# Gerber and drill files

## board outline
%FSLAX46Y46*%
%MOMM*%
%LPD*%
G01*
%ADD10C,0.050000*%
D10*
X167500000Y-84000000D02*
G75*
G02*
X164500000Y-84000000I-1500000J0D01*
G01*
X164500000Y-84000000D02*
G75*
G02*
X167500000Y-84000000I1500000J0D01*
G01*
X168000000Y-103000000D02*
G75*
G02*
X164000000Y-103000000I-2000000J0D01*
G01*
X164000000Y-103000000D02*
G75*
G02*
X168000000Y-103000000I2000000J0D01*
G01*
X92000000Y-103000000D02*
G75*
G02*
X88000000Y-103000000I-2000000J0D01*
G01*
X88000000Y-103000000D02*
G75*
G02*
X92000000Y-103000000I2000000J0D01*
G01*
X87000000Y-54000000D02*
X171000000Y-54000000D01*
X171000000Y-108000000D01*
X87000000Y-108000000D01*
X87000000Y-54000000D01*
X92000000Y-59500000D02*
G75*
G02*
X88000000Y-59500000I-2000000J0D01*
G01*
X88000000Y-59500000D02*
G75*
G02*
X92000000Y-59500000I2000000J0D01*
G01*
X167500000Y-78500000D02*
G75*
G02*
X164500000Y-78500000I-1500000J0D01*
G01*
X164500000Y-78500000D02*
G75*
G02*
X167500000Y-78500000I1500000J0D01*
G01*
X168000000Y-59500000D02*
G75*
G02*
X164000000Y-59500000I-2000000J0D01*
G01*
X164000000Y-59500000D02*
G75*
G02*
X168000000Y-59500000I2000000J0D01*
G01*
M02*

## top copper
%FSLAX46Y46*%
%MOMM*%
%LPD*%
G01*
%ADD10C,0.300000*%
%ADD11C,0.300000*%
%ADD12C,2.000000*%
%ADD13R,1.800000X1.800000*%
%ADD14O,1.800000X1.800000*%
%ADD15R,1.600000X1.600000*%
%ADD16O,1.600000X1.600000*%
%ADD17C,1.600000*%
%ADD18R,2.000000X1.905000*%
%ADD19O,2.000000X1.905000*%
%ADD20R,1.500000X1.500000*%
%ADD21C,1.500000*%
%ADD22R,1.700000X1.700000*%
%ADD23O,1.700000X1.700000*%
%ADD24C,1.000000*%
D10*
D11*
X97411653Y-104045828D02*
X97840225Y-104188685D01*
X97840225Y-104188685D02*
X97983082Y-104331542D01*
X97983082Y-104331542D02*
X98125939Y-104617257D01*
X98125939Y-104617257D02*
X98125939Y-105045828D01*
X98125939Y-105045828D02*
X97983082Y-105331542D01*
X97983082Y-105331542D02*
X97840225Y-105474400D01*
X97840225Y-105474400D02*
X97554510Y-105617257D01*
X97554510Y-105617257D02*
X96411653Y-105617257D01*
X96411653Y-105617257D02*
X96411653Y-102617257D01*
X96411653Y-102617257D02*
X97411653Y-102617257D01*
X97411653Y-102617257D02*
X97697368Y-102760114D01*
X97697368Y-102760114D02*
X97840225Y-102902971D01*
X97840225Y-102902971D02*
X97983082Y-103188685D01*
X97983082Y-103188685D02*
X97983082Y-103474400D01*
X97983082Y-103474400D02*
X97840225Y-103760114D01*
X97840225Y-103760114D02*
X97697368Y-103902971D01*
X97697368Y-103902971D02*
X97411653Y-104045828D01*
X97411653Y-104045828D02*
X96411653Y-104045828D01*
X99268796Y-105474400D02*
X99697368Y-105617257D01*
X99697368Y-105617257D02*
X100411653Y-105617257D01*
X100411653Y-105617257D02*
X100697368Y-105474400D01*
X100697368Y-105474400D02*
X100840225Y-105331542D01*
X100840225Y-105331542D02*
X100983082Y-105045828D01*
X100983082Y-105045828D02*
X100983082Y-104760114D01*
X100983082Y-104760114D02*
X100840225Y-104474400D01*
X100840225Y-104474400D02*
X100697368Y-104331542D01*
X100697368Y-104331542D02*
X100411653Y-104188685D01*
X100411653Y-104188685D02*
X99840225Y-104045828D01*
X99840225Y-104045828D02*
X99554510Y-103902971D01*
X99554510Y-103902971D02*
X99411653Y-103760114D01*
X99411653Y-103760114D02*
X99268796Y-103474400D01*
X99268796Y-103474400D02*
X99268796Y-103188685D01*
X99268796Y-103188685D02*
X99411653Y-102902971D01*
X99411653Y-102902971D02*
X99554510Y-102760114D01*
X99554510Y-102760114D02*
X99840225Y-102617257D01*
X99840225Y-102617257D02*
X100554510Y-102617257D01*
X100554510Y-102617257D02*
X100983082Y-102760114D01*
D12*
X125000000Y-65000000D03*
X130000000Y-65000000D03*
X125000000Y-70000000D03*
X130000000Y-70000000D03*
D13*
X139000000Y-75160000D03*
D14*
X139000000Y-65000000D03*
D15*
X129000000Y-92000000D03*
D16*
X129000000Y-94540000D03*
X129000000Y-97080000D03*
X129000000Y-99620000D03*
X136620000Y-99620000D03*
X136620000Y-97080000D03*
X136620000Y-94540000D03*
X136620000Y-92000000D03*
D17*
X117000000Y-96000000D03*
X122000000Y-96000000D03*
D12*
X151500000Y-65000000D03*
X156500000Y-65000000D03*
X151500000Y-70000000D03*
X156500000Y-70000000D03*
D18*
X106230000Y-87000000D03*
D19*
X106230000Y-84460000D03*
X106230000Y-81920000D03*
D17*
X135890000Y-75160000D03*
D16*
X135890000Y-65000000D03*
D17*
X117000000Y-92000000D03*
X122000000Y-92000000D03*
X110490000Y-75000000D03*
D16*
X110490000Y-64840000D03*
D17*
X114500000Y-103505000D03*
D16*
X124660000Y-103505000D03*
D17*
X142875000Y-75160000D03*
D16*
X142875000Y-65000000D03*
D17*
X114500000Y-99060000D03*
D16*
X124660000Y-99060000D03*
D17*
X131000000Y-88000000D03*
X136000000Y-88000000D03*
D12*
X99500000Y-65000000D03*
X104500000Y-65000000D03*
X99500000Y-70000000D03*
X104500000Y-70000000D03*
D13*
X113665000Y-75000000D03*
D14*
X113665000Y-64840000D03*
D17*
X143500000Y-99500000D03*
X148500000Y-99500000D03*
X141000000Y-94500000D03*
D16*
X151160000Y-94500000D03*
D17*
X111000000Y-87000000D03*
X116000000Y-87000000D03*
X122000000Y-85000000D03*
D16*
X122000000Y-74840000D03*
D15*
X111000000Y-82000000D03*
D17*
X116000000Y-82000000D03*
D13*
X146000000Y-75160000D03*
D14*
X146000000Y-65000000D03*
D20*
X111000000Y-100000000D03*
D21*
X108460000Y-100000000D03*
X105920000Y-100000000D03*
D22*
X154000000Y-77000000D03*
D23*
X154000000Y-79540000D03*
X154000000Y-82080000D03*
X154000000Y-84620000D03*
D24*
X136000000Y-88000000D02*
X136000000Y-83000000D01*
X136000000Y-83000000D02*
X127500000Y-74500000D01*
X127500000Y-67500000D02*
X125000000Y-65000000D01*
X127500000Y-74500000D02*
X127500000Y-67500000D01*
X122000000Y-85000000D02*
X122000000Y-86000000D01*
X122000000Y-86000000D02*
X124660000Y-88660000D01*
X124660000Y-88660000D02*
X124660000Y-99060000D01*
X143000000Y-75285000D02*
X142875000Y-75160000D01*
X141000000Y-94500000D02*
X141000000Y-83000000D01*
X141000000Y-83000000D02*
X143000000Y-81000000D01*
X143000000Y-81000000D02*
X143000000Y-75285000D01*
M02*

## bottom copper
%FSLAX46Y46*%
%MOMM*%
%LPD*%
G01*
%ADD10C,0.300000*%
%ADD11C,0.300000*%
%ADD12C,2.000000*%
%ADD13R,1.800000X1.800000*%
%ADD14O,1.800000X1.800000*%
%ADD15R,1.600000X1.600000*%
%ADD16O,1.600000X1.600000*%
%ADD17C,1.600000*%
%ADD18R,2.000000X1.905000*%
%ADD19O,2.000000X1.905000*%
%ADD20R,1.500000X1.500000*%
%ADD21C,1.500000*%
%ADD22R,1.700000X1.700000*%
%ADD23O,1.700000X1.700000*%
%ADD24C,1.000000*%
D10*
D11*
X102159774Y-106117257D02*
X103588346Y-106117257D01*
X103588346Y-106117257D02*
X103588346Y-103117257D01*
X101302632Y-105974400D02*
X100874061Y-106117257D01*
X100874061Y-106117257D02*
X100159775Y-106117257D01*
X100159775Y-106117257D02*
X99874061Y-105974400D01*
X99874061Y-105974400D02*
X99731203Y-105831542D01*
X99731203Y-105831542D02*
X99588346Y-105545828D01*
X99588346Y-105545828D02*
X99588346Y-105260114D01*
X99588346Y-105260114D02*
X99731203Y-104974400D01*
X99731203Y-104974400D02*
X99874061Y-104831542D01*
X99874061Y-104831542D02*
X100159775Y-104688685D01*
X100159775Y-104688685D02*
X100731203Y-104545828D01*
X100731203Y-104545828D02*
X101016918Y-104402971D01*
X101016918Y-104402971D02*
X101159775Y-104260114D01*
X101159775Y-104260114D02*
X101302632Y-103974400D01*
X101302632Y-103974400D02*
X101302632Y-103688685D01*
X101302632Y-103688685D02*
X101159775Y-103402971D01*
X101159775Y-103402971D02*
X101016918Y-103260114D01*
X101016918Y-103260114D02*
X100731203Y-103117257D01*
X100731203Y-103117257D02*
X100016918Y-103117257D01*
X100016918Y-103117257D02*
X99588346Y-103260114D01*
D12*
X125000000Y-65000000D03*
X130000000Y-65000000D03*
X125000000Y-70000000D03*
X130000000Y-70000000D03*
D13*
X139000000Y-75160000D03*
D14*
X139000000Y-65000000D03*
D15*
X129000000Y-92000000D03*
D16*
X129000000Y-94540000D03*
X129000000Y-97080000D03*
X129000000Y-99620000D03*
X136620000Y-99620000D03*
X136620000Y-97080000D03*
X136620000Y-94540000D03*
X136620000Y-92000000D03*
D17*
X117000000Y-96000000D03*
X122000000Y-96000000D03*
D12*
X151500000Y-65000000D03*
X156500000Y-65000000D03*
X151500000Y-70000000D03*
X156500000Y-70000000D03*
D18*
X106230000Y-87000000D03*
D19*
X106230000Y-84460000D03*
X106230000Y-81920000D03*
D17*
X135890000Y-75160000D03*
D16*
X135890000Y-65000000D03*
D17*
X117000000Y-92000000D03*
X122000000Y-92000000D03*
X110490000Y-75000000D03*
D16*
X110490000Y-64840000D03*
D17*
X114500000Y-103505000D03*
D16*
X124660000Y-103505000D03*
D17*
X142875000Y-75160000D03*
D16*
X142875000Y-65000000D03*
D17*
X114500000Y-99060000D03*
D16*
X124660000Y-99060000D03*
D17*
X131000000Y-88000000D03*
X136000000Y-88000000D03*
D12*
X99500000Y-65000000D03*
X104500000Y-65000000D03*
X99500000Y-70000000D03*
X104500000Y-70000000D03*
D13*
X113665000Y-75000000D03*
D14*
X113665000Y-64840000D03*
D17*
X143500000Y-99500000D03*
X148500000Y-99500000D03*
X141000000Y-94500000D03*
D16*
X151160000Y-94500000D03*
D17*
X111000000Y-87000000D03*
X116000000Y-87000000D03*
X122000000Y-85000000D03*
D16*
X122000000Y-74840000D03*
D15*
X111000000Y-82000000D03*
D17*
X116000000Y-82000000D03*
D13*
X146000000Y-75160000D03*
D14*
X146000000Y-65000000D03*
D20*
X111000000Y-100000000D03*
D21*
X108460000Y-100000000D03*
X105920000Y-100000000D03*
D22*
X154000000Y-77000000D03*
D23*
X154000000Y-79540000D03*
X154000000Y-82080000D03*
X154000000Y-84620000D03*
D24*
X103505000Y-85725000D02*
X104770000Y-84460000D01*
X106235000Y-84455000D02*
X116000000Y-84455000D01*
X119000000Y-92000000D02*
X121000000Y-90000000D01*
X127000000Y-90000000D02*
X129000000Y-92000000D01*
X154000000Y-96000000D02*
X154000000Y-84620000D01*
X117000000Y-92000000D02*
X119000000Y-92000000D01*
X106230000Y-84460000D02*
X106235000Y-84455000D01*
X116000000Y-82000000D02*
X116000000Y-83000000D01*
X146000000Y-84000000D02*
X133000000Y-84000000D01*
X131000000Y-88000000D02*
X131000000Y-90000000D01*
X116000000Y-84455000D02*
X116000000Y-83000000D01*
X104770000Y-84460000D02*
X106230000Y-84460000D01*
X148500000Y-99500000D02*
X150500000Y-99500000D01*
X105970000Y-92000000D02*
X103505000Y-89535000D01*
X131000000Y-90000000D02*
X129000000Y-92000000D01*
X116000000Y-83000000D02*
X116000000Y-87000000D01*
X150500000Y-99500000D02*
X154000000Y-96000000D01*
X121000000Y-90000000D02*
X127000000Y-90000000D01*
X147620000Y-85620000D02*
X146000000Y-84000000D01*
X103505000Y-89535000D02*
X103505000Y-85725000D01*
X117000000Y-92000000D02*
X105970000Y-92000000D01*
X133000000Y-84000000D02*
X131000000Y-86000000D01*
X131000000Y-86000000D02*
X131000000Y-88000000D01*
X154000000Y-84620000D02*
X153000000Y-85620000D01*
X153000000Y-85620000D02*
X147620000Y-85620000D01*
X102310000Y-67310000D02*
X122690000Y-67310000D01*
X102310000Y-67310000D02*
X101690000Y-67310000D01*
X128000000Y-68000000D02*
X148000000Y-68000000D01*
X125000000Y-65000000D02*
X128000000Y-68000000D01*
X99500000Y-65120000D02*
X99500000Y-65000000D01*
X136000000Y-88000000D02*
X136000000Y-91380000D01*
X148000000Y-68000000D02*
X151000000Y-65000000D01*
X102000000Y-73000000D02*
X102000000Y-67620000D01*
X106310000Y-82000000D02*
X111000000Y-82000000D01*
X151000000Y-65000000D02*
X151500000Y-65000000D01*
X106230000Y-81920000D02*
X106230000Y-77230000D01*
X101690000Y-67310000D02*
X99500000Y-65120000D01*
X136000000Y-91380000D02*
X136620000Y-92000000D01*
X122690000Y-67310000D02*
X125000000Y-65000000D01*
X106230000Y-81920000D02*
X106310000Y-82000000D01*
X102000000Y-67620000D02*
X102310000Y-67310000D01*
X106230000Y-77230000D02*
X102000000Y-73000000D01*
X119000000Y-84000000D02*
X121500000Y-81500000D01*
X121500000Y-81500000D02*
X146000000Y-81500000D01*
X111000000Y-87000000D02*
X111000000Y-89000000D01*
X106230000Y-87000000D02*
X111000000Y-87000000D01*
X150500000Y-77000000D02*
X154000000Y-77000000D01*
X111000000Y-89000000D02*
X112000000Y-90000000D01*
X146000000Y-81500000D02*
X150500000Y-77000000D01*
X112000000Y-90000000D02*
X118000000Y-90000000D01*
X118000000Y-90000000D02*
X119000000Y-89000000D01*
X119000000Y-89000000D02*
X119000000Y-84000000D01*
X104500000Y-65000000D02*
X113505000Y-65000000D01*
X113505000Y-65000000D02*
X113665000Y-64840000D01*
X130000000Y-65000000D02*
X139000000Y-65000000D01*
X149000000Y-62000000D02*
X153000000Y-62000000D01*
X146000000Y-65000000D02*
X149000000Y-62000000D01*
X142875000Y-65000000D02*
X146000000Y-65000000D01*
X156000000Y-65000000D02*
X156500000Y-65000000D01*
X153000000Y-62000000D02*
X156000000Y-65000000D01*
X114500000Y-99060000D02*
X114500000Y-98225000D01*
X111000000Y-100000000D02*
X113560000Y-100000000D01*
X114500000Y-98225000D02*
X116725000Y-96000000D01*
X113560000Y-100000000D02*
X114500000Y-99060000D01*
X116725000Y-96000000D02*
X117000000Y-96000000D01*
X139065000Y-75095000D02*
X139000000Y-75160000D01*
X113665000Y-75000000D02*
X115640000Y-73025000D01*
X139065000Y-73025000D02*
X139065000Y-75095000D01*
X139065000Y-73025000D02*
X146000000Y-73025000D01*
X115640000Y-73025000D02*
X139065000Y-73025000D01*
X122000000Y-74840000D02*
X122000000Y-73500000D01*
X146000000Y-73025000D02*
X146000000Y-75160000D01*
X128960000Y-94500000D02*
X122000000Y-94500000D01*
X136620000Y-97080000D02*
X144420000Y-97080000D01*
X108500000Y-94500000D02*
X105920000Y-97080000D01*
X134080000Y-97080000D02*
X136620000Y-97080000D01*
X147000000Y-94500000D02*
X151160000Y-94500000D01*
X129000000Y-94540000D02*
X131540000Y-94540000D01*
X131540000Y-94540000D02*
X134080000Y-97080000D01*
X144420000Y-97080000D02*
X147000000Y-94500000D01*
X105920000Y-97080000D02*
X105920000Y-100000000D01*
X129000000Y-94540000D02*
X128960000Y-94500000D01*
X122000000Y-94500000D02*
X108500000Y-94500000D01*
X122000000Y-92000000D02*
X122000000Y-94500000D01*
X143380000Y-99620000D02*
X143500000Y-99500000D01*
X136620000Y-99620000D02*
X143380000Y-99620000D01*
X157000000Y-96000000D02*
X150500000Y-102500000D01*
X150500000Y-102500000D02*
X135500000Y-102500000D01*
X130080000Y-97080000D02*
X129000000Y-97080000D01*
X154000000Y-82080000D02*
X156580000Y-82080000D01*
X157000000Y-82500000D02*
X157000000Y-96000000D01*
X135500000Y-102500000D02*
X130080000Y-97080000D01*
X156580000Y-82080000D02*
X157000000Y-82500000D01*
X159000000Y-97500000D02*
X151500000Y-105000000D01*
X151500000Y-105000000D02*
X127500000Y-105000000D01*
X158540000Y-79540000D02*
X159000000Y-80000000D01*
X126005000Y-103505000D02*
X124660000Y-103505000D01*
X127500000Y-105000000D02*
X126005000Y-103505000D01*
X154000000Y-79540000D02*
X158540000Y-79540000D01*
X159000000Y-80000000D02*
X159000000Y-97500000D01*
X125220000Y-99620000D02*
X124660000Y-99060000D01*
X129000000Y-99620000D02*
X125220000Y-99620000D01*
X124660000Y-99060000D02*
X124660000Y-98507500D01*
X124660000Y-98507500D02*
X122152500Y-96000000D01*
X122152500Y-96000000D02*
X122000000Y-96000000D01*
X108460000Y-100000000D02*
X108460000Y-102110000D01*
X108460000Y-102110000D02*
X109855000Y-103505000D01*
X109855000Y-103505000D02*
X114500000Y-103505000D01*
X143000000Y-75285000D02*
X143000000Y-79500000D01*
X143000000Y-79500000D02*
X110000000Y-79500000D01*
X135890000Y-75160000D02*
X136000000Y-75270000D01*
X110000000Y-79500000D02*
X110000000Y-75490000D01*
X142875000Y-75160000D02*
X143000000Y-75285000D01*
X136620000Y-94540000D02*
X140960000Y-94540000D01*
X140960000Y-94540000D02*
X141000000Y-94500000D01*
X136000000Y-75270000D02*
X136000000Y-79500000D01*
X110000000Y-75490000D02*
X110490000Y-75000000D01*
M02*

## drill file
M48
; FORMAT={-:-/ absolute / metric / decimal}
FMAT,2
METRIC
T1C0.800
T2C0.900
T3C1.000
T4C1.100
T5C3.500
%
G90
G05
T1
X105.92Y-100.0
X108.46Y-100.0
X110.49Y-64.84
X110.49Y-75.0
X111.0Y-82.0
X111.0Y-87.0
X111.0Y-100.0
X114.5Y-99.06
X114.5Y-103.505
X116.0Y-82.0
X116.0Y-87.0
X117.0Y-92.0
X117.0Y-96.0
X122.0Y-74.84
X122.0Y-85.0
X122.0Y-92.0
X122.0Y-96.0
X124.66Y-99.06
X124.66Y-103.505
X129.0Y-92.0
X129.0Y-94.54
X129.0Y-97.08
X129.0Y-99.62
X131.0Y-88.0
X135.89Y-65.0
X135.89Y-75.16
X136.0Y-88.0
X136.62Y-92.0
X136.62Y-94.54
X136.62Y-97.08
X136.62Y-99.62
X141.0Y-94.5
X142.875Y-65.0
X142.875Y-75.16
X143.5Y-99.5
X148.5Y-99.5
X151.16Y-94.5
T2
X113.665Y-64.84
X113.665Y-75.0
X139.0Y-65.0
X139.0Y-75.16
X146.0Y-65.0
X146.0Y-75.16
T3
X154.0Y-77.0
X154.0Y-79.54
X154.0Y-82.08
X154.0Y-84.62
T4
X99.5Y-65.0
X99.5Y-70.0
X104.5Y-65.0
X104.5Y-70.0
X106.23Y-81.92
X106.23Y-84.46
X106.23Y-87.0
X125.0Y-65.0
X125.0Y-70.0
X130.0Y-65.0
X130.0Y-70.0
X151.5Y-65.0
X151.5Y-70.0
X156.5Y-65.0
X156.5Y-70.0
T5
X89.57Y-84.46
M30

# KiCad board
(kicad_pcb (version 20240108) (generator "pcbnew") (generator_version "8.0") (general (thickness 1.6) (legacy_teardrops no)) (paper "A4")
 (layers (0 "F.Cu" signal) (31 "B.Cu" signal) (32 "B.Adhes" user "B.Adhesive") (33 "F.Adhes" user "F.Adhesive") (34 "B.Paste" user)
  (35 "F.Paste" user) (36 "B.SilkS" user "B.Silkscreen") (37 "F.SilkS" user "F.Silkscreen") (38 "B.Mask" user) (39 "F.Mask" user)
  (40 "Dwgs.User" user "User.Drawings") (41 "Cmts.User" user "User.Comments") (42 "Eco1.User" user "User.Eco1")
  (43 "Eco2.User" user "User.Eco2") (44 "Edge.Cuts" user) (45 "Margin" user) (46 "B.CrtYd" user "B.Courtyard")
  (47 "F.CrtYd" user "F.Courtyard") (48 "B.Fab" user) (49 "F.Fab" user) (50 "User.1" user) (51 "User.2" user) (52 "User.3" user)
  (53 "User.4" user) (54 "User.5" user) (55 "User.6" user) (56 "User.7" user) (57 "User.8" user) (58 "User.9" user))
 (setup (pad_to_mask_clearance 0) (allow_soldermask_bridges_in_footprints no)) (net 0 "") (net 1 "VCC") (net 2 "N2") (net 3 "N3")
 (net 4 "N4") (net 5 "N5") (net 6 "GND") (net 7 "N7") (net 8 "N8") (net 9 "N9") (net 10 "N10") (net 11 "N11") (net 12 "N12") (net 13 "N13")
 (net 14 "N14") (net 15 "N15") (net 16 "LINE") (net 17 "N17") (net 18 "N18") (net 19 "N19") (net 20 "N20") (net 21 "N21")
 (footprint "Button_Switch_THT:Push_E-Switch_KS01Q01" (layer "F.Cu") (at 125 65)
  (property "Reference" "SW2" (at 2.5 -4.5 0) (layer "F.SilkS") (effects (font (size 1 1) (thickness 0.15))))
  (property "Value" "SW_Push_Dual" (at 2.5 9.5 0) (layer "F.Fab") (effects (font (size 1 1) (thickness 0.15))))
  (pad "1" thru_hole circle (at 0 0) (size 2 2) (drill 1.1) (layers "*.Cu" "*.Mask") (remove_unused_layers no) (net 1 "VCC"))
  (pad "2" thru_hole circle (at 5 0) (size 2 2) (drill 1.1) (layers "*.Cu" "*.Mask") (remove_unused_layers no) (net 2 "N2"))
  (pad "3" thru_hole circle (at 0 5) (size 2 2) (drill 1.1) (layers "*.Cu" "*.Mask") (remove_unused_layers no) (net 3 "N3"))
  (pad "4" thru_hole circle (at 5 5) (size 2 2) (drill 1.1) (layers "*.Cu" "*.Mask") (remove_unused_layers no) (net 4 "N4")))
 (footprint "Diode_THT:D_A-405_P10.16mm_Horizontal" (layer "F.Cu") (at 139 75.16 90)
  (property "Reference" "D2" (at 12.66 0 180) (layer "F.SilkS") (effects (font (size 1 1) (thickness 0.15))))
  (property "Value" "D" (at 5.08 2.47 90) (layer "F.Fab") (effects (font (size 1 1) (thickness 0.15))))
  (pad "1" thru_hole rect (at 0 0 90) (size 1.8 1.8) (drill 0.9) (layers "*.Cu" "*.Mask") (remove_unused_layers no) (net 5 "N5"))
  (pad "2" thru_hole oval (at 10.16 0 90) (size 1.8 1.8) (drill 0.9) (layers "*.Cu" "*.Mask") (remove_unused_layers no) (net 2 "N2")))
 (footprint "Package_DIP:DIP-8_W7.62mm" (layer "F.Cu") (at 129 92)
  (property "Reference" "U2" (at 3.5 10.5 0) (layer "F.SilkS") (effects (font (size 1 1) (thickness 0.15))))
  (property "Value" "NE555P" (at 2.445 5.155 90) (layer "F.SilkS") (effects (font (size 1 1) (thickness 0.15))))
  (pad "1" thru_hole rect (at 0 0) (size 1.6 1.6) (drill 0.8) (layers "*.Cu" "*.Mask") (remove_unused_layers no) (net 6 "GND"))
  (pad "2" thru_hole oval (at 0 2.54) (size 1.6 1.6) (drill 0.8) (layers "*.Cu" "*.Mask") (remove_unused_layers no) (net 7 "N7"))
  (pad "3" thru_hole oval (at 0 5.08) (size 1.6 1.6) (drill 0.8) (layers "*.Cu" "*.Mask") (remove_unused_layers no) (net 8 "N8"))
  (pad "4" thru_hole oval (at 0 7.62) (size 1.6 1.6) (drill 0.8) (layers "*.Cu" "*.Mask") (remove_unused_layers no) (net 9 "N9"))
  (pad "5" thru_hole oval (at 7.62 7.62) (size 1.6 1.6) (drill 0.8) (layers "*.Cu" "*.Mask") (remove_unused_layers no) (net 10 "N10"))
  (pad "6" thru_hole oval (at 7.62 5.08) (size 1.6 1.6) (drill 0.8) (layers "*.Cu" "*.Mask") (remove_unused_layers no) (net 7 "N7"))
  (pad "7" thru_hole oval (at 7.62 2.54) (size 1.6 1.6) (drill 0.8) (layers "*.Cu" "*.Mask") (remove_unused_layers no) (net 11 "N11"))
  (pad "8" thru_hole oval (at 7.62 0) (size 1.6 1.6) (drill 0.8) (layers "*.Cu" "*.Mask") (remove_unused_layers no) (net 1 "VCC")))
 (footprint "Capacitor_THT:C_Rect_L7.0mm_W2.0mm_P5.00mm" (layer "F.Cu") (at 117 96)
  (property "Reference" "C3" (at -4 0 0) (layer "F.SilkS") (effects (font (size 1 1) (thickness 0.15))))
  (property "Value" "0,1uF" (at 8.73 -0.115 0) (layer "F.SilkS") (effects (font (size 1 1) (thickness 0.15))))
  (pad "1" thru_hole circle (at 0 0) (size 1.6 1.6) (drill 0.8) (layers "*.Cu" "*.Mask") (remove_unused_layers no) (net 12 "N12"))
  (pad "2" thru_hole circle (at 5 0) (size 1.6 1.6) (drill 0.8) (layers "*.Cu" "*.Mask") (remove_unused_layers no) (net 9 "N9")))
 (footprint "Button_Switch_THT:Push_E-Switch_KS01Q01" (layer "F.Cu") (at 151.5 65)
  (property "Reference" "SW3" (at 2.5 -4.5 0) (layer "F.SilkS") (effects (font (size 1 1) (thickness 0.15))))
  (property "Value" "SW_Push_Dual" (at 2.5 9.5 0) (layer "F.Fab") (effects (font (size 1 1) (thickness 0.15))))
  (pad "1" thru_hole circle (at 0 0) (size 2 2) (drill 1.1) (layers "*.Cu" "*.Mask") (remove_unused_layers no) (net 1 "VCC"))
  (pad "2" thru_hole circle (at 5 0) (size 2 2) (drill 1.1) (layers "*.Cu" "*.Mask") (remove_unused_layers no) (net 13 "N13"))
  (pad "3" thru_hole circle (at 0 5) (size 2 2) (drill 1.1) (layers "*.Cu" "*.Mask") (remove_unused_layers no) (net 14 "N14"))
  (pad "4" thru_hole circle (at 5 5) (size 2 2) (drill 1.1) (layers "*.Cu" "*.Mask") (remove_unused_layers no) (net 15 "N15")))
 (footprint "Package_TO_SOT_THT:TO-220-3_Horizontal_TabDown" (layer "F.Cu") (at 106.23 87 90)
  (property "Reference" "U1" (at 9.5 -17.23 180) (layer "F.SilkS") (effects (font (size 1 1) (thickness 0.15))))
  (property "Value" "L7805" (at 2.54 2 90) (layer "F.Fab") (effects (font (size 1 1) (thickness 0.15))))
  (pad "" np_thru_hole circle (at 2.54 -16.66 90) (size 3.5 3.5) (drill 3.5) (layers "*.Cu" "*.Mask"))
  (pad "1" thru_hole rect (at 0 0 90) (size 1.905 2) (drill 1.1) (layers "*.Cu" "*.Mask") (remove_unused_layers no) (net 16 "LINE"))
  (pad "2" thru_hole oval (at 2.54 0 90) (size 1.905 2) (drill 1.1) (layers "*.Cu" "*.Mask") (remove_unused_layers no) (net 6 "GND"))
  (pad "3" thru_hole oval (at 5.08 0 90) (size 1.905 2) (drill 1.1) (layers "*.Cu" "*.Mask") (remove_unused_layers no) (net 1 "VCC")))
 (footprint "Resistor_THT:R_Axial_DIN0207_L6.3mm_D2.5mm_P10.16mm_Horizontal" (layer "F.Cu") (at 135.89 75.16 90)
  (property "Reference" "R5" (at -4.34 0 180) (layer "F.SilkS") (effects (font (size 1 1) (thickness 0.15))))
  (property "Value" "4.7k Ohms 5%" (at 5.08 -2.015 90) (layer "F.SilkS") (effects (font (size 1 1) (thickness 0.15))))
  (pad "1" thru_hole circle (at 0 0 90) (size 1.6 1.6) (drill 0.8) (layers "*.Cu" "*.Mask") (remove_unused_layers no) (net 11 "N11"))
  (pad "2" thru_hole oval (at 10.16 0 90) (size 1.6 1.6) (drill 0.8) (layers "*.Cu" "*.Mask") (remove_unused_layers no) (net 2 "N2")))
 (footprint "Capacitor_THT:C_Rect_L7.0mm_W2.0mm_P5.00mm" (layer "F.Cu") (at 117 92)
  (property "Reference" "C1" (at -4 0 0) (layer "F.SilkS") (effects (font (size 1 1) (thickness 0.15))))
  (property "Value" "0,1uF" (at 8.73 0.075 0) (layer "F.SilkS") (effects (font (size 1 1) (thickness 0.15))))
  (pad "1" thru_hole circle (at 0 0) (size 1.6 1.6) (drill 0.8) (layers "*.Cu" "*.Mask") (remove_unused_layers no) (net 6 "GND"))
  (pad "2" thru_hole circle (at 5 0) (size 1.6 1.6) (drill 0.8) (layers "*.Cu" "*.Mask") (remove_unused_layers no) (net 7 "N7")))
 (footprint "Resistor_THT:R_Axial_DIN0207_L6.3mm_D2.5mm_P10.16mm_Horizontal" (layer "F.Cu") (at 110.49 75 90)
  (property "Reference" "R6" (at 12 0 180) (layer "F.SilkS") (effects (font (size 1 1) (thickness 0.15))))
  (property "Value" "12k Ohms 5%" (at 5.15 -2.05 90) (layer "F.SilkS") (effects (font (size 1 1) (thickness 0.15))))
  (pad "1" thru_hole circle (at 0 0 90) (size 1.6 1.6) (drill 0.8) (layers "*.Cu" "*.Mask") (remove_unused_layers no) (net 11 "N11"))
  (pad "2" thru_hole oval (at 10.16 0 90) (size 1.6 1.6) (drill 0.8) (layers "*.Cu" "*.Mask") (remove_unused_layers no) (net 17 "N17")))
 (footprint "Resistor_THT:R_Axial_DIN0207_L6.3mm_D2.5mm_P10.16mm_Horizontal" (layer "F.Cu") (at 114.5 103.505)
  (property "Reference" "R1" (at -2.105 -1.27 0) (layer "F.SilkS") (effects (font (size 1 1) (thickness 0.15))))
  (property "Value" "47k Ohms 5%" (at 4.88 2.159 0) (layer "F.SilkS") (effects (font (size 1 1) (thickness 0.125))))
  (pad "1" thru_hole circle (at 0 0) (size 1.6 1.6) (drill 0.8) (layers "*.Cu" "*.Mask") (remove_unused_layers no) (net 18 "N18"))
  (pad "2" thru_hole oval (at 10.16 0) (size 1.6 1.6) (drill 0.8) (layers "*.Cu" "*.Mask") (remove_unused_layers no) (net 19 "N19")))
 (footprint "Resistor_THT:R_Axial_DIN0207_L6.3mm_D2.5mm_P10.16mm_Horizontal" (layer "F.Cu") (at 142.875 75.16 90)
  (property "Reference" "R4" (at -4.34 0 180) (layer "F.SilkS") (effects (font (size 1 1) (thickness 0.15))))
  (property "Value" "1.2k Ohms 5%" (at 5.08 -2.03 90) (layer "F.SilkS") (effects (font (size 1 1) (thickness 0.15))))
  (pad "1" thru_hole circle (at 0 0 90) (size 1.6 1.6) (drill 0.8) (layers "*.Cu" "*.Mask") (remove_unused_layers no) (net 11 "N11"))
  (pad "2" thru_hole oval (at 10.16 0 90) (size 1.6 1.6) (drill 0.8) (layers "*.Cu" "*.Mask") (remove_unused_layers no) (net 13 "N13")))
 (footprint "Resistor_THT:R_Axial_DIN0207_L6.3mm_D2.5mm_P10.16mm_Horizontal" (layer "F.Cu") (at 114.5 99.06)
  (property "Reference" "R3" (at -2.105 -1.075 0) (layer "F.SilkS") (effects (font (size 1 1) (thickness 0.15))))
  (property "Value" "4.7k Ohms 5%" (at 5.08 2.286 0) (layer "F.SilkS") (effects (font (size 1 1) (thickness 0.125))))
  (pad "1" thru_hole circle (at 0 0) (size 1.6 1.6) (drill 0.8) (layers "*.Cu" "*.Mask") (remove_unused_layers no) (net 12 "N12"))
  (pad "2" thru_hole oval (at 10.16 0) (size 1.6 1.6) (drill 0.8) (layers "*.Cu" "*.Mask") (remove_unused_layers no) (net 9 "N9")))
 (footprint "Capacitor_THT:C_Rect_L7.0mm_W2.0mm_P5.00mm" (layer "F.Cu") (at 131 88)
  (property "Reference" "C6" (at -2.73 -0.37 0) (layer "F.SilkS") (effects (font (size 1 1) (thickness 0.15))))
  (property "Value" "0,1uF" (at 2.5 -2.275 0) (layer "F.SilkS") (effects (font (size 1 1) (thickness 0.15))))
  (pad "1" thru_hole circle (at 0 0) (size 1.6 1.6) (drill 0.8) (layers "*.Cu" "*.Mask") (remove_unused_layers no) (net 6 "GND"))
  (pad "2" thru_hole circle (at 5 0) (size 1.6 1.6) (drill 0.8) (layers "*.Cu" "*.Mask") (remove_unused_layers no) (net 1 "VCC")))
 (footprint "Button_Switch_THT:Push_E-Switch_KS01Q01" (layer "F.Cu") (at 99.5 65)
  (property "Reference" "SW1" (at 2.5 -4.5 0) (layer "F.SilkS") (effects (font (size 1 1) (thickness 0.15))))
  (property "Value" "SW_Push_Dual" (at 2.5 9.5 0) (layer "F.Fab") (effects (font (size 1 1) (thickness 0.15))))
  (pad "1" thru_hole circle (at 0 0) (size 2 2) (drill 1.1) (layers "*.Cu" "*.Mask") (remove_unused_layers no) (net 1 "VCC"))
  (pad "2" thru_hole circle (at 5 0) (size 2 2) (drill 1.1) (layers "*.Cu" "*.Mask") (remove_unused_layers no) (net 17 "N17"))
  (pad "3" thru_hole circle (at 0 5) (size 2 2) (drill 1.1) (layers "*.Cu" "*.Mask") (remove_unused_layers no) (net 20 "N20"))
  (pad "4" thru_hole circle (at 5 5) (size 2 2) (drill 1.1) (layers "*.Cu" "*.Mask") (remove_unused_layers no) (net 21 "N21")))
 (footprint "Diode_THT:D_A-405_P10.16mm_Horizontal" (layer "F.Cu") (at 113.665 75 90)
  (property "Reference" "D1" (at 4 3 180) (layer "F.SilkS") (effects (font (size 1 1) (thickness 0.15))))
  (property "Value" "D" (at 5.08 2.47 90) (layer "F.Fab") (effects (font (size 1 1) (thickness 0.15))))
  (pad "1" thru_hole rect (at 0 0 90) (size 1.8 1.8) (drill 0.9) (layers "*.Cu" "*.Mask") (remove_unused_layers no) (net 5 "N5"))
  (pad "2" thru_hole oval (at 10.16 0 90) (size 1.8 1.8) (drill 0.9) (layers "*.Cu" "*.Mask") (remove_unused_layers no) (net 17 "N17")))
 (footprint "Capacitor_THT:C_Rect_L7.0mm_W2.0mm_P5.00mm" (layer "F.Cu") (at 143.5 99.5)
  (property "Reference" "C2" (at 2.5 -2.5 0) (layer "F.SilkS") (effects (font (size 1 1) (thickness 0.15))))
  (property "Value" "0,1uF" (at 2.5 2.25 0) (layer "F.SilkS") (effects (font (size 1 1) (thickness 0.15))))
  (pad "1" thru_hole circle (at 0 0) (size 1.6 1.6) (drill 0.8) (layers "*.Cu" "*.Mask") (remove_unused_layers no) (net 10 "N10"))
  (pad "2" thru_hole circle (at 5 0) (size 1.6 1.6) (drill 0.8) (layers "*.Cu" "*.Mask") (remove_unused_layers no) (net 6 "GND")))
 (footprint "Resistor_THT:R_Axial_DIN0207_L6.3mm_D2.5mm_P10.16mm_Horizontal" (layer "F.Cu") (at 141 94.5)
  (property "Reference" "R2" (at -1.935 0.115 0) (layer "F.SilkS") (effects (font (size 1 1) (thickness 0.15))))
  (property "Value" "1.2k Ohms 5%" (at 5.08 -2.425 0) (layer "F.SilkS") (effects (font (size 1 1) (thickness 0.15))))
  (pad "1" thru_hole circle (at 0 0) (size 1.6 1.6) (drill 0.8) (layers "*.Cu" "*.Mask") (remove_unused_layers no) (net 11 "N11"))
  (pad "2" thru_hole oval (at 10.16 0) (size 1.6 1.6) (drill 0.8) (layers "*.Cu" "*.Mask") (remove_unused_layers no) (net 7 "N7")))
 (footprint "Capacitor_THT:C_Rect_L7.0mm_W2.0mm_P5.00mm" (layer "F.Cu") (at 111 87)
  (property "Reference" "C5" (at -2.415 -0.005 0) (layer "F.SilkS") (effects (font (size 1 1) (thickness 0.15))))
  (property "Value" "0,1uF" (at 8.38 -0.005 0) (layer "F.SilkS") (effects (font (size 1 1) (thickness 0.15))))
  (pad "1" thru_hole circle (at 0 0) (size 1.6 1.6) (drill 0.8) (layers "*.Cu" "*.Mask") (remove_unused_layers no) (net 16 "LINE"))
  (pad "2" thru_hole circle (at 5 0) (size 1.6 1.6) (drill 0.8) (layers "*.Cu" "*.Mask") (remove_unused_layers no) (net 6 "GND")))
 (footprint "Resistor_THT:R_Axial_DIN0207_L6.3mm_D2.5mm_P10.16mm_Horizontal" (layer "F.Cu") (at 122 85 90)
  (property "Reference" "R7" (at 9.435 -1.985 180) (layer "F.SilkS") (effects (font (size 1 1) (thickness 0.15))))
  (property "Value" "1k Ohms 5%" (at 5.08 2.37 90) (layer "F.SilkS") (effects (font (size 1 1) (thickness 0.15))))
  (pad "1" thru_hole circle (at 0 0 90) (size 1.6 1.6) (drill 0.8) (layers "*.Cu" "*.Mask") (remove_unused_layers no) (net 9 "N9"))
  (pad "2" thru_hole oval (at 10.16 0 90) (size 1.6 1.6) (drill 0.8) (layers "*.Cu" "*.Mask") (remove_unused_layers no) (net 5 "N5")))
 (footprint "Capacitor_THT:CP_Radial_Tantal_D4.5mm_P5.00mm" (layer "F.Cu") (at 111 82)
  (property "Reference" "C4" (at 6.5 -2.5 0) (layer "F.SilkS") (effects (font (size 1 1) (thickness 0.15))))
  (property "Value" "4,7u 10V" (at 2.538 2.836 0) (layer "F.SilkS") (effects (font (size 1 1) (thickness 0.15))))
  (pad "1" thru_hole rect (at 0 0) (size 1.6 1.6) (drill 0.8) (layers "*.Cu" "*.Mask") (remove_unused_layers no) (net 1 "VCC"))
  (pad "2" thru_hole circle (at 5 0) (size 1.6 1.6) (drill 0.8) (layers "*.Cu" "*.Mask") (remove_unused_layers no) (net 6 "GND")))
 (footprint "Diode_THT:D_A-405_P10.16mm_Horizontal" (layer "F.Cu") (at 146 75.16 90)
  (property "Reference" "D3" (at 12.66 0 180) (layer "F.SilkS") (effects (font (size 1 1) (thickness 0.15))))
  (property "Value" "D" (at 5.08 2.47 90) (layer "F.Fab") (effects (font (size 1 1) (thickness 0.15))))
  (pad "1" thru_hole rect (at 0 0 90) (size 1.8 1.8) (drill 0.9) (layers "*.Cu" "*.Mask") (remove_unused_layers no) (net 5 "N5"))
  (pad "2" thru_hole oval (at 10.16 0 90) (size 1.8 1.8) (drill 0.9) (layers "*.Cu" "*.Mask") (remove_unused_layers no) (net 13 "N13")))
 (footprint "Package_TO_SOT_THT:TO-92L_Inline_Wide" (layer "F.Cu") (at 111 100 180)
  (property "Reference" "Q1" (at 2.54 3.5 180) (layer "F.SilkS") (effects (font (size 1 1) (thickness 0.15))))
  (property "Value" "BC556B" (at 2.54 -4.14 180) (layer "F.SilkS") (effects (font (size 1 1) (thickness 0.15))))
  (pad "1" thru_hole rect (at 0 0 180) (size 1.5 1.5) (drill 0.8) (layers "*.Cu" "*.Mask") (remove_unused_layers no) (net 12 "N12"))
  (pad "2" thru_hole circle (at 2.54 0 180) (size 1.5 1.5) (drill 0.8) (layers "*.Cu" "*.Mask") (remove_unused_layers no) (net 18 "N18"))
  (pad "3" thru_hole circle (at 5.08 0 180) (size 1.5 1.5) (drill 0.8) (layers "*.Cu" "*.Mask") (remove_unused_layers no) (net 7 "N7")))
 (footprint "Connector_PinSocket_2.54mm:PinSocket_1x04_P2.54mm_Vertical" (layer "F.Cu") (at 154 77)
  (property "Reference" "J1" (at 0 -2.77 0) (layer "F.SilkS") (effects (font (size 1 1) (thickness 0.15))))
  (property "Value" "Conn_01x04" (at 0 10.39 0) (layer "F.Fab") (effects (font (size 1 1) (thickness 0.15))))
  (pad "1" thru_hole rect (at 0 0) (size 1.7 1.7) (drill 1) (layers "*.Cu" "*.Mask") (remove_unused_layers no) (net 16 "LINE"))
  (pad "2" thru_hole oval (at 0 2.54) (size 1.7 1.7) (drill 1) (layers "*.Cu" "*.Mask") (remove_unused_layers no) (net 19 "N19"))
  (pad "3" thru_hole oval (at 0 5.08) (size 1.7 1.7) (drill 1) (layers "*.Cu" "*.Mask") (remove_unused_layers no) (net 8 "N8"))
  (pad "4" thru_hole oval (at 0 7.62) (size 1.7 1.7) (drill 1) (layers "*.Cu" "*.Mask") (remove_unused_layers no) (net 6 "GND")))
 (gr_circle (center 166 84) (end 167.5 84) (stroke (width 0.05) (type default)) (fill none) (layer "Edge.Cuts"))
 (gr_circle (center 166 103) (end 166 101) (stroke (width 0.05) (type default)) (fill none) (layer "Edge.Cuts"))
 (gr_circle (center 90 103) (end 90 101) (stroke (width 0.05) (type default)) (fill none) (layer "Edge.Cuts"))
 (gr_rect (start 87 54) (end 171 108) (stroke (width 0.05) (type default)) (fill none) (layer "Edge.Cuts"))
 (gr_circle (center 90 59.5) (end 90 57.5) (stroke (width 0.05) (type default)) (fill none) (layer "Edge.Cuts"))
 (gr_circle (center 166 78.5) (end 167.5 78.5) (stroke (width 0.05) (type default)) (fill none) (layer "Edge.Cuts"))
 (gr_circle (center 166 59.5) (end 166 57.5) (stroke (width 0.05) (type default)) (fill none) (layer "Edge.Cuts"))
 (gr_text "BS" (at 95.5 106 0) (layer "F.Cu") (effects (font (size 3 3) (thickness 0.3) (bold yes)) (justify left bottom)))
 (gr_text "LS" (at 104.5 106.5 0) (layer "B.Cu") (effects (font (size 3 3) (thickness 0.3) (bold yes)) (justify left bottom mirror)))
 (segment (start 103.505 85.725) (end 104.77 84.46) (width 1) (layer "B.Cu") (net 6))
 (segment (start 106.235 84.455) (end 116 84.455) (width 1) (layer "B.Cu") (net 6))
 (segment (start 119 92) (end 121 90) (width 1) (layer "B.Cu") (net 6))
 (segment (start 127 90) (end 129 92) (width 1) (layer "B.Cu") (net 6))
 (segment (start 154 96) (end 154 84.62) (width 1) (layer "B.Cu") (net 6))
 (segment (start 117 92) (end 119 92) (width 1) (layer "B.Cu") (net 6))
 (segment (start 106.23 84.46) (end 106.235 84.455) (width 1) (layer "B.Cu") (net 6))
 (segment (start 116 82) (end 116 83) (width 1) (layer "B.Cu") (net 6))
 (segment (start 146 84) (end 133 84) (width 1) (layer "B.Cu") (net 6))
 (segment (start 131 88) (end 131 90) (width 1) (layer "B.Cu") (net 6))
 (segment (start 116 84.455) (end 116 83) (width 1) (layer "B.Cu") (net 6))
 (segment (start 104.77 84.46) (end 106.23 84.46) (width 1) (layer "B.Cu") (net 6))
 (segment (start 148.5 99.5) (end 150.5 99.5) (width 1) (layer "B.Cu") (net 6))
 (segment (start 105.97 92) (end 103.505 89.535) (width 1) (layer "B.Cu") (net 6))
 (segment (start 131 90) (end 129 92) (width 1) (layer "B.Cu") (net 6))
 (segment (start 116 83) (end 116 87) (width 1) (layer "B.Cu") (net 6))
 (segment (start 150.5 99.5) (end 154 96) (width 1) (layer "B.Cu") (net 6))
 (segment (start 121 90) (end 127 90) (width 1) (layer "B.Cu") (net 6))
 (segment (start 147.62 85.62) (end 146 84) (width 1) (layer "B.Cu") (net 6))
 (segment (start 103.505 89.535) (end 103.505 85.725) (width 1) (layer "B.Cu") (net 6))
 (segment (start 117 92) (end 105.97 92) (width 1) (layer "B.Cu") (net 6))
 (segment (start 133 84) (end 131 86) (width 1) (layer "B.Cu") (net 6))
 (segment (start 131 86) (end 131 88) (width 1) (layer "B.Cu") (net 6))
 (segment (start 154 84.62) (end 153 85.62) (width 1) (layer "B.Cu") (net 6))
 (segment (start 153 85.62) (end 147.62 85.62) (width 1) (layer "B.Cu") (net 6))
 (segment (start 136 88) (end 136 83) (width 1) (layer "F.Cu") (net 1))
 (segment (start 136 83) (end 127.5 74.5) (width 1) (layer "F.Cu") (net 1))
 (segment (start 127.5 67.5) (end 125 65) (width 1) (layer "F.Cu") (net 1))
 (segment (start 127.5 74.5) (end 127.5 67.5) (width 1) (layer "F.Cu") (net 1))
 (segment (start 102.31 67.31) (end 122.69 67.31) (width 1) (layer "B.Cu") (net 1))
 (segment (start 102.31 67.31) (end 101.69 67.31) (width 1) (layer "B.Cu") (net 1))
 (segment (start 128 68) (end 148 68) (width 1) (layer "B.Cu") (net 1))
 (segment (start 125 65) (end 128 68) (width 1) (layer "B.Cu") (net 1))
 (segment (start 99.5 65.12) (end 99.5 65) (width 1) (layer "B.Cu") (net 1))
 (segment (start 136 88) (end 136 91.38) (width 1) (layer "B.Cu") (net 1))
 (segment (start 148 68) (end 151 65) (width 1) (layer "B.Cu") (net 1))
 (segment (start 102 73) (end 102 67.62) (width 1) (layer "B.Cu") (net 1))
 (segment (start 106.31 82) (end 111 82) (width 1) (layer "B.Cu") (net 1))
 (segment (start 151 65) (end 151.5 65) (width 1) (layer "B.Cu") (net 1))
 (segment (start 106.23 81.92) (end 106.23 77.23) (width 1) (layer "B.Cu") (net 1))
 (segment (start 101.69 67.31) (end 99.5 65.12) (width 1) (layer "B.Cu") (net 1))
 (segment (start 136 91.38) (end 136.62 92) (width 1) (layer "B.Cu") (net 1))
 (segment (start 122.69 67.31) (end 125 65) (width 1) (layer "B.Cu") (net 1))
 (segment (start 106.23 81.92) (end 106.31 82) (width 1) (layer "B.Cu") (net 1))
 (segment (start 102 67.62) (end 102.31 67.31) (width 1) (layer "B.Cu") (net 1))
 (segment (start 106.23 77.23) (end 102 73) (width 1) (layer "B.Cu") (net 1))
 (segment (start 119 84) (end 121.5 81.5) (width 1) (layer "B.Cu") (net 16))
 (segment (start 121.5 81.5) (end 146 81.5) (width 1) (layer "B.Cu") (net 16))
 (segment (start 111 87) (end 111 89) (width 1) (layer "B.Cu") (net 16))
 (segment (start 106.23 87) (end 111 87) (width 1) (layer "B.Cu") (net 16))
 (segment (start 150.5 77) (end 154 77) (width 1) (layer "B.Cu") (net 16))
 (segment (start 111 89) (end 112 90) (width 1) (layer "B.Cu") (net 16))
 (segment (start 146 81.5) (end 150.5 77) (width 1) (layer "B.Cu") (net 16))
 (segment (start 112 90) (end 118 90) (width 1) (layer "B.Cu") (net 16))
 (segment (start 118 90) (end 119 89) (width 1) (layer "B.Cu") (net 16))
 (segment (start 119 89) (end 119 84) (width 1) (layer "B.Cu") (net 16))
 (segment (start 104.5 65) (end 113.505 65) (width 1) (layer "B.Cu") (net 17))
 (segment (start 113.505 65) (end 113.665 64.84) (width 1) (layer "B.Cu") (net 17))
 (segment (start 130 65) (end 139 65) (width 1) (layer "B.Cu") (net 2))
 (segment (start 149 62) (end 153 62) (width 1) (layer "B.Cu") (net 13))
 (segment (start 146 65) (end 149 62) (width 1) (layer "B.Cu") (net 13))
 (segment (start 142.875 65) (end 146 65) (width 1) (layer "B.Cu") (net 13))
 (segment (start 156 65) (end 156.5 65) (width 1) (layer "B.Cu") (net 13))
 (segment (start 153 62) (end 156 65) (width 1) (layer "B.Cu") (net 13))
 (segment (start 114.5 99.06) (end 114.5 98.225) (width 1) (layer "B.Cu") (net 12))
 (segment (start 111 100) (end 113.56 100) (width 1) (layer "B.Cu") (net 12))
 (segment (start 114.5 98.225) (end 116.725 96) (width 1) (layer "B.Cu") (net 12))
 (segment (start 113.56 100) (end 114.5 99.06) (width 1) (layer "B.Cu") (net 12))
 (segment (start 116.725 96) (end 117 96) (width 1) (layer "B.Cu") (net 12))
 (segment (start 139.065 75.095) (end 139 75.16) (width 1) (layer "B.Cu") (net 5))
 (segment (start 113.665 75) (end 115.64 73.025) (width 1) (layer "B.Cu") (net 5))
 (segment (start 139.065 73.025) (end 139.065 75.095) (width 1) (layer "B.Cu") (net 5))
 (segment (start 139.065 73.025) (end 146 73.025) (width 1) (layer "B.Cu") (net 5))
 (segment (start 115.64 73.025) (end 139.065 73.025) (width 1) (layer "B.Cu") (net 5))
 (segment (start 122 74.84) (end 122 73.5) (width 1) (layer "B.Cu") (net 5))
 (segment (start 146 73.025) (end 146 75.16) (width 1) (layer "B.Cu") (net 5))
 (segment (start 128.96 94.5) (end 122 94.5) (width 1) (layer "B.Cu") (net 7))
 (segment (start 136.62 97.08) (end 144.42 97.08) (width 1) (layer "B.Cu") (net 7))
 (segment (start 108.5 94.5) (end 105.92 97.08) (width 1) (layer "B.Cu") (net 7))
 (segment (start 134.08 97.08) (end 136.62 97.08) (width 1) (layer "B.Cu") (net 7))
 (segment (start 147 94.5) (end 151.16 94.5) (width 1) (layer "B.Cu") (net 7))
 (segment (start 129 94.54) (end 131.54 94.54) (width 1) (layer "B.Cu") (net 7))
 (segment (start 131.54 94.54) (end 134.08 97.08) (width 1) (layer "B.Cu") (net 7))
 (segment (start 144.42 97.08) (end 147 94.5) (width 1) (layer "B.Cu") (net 7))
 (segment (start 105.92 97.08) (end 105.92 100) (width 1) (layer "B.Cu") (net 7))
 (segment (start 129 94.54) (end 128.96 94.5) (width 1) (layer "B.Cu") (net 7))
 (segment (start 122 94.5) (end 108.5 94.5) (width 1) (layer "B.Cu") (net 7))
 (segment (start 122 92) (end 122 94.5) (width 1) (layer "B.Cu") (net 7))
 (segment (start 143.38 99.62) (end 143.5 99.5) (width 1) (layer "B.Cu") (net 10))
 (segment (start 136.62 99.62) (end 143.38 99.62) (width 1) (layer "B.Cu") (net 10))
 (segment (start 157 96) (end 150.5 102.5) (width 1) (layer "B.Cu") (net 8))
 (segment (start 150.5 102.5) (end 135.5 102.5) (width 1) (layer "B.Cu") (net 8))
 (segment (start 130.08 97.08) (end 129 97.08) (width 1) (layer "B.Cu") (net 8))
 (segment (start 154 82.08) (end 156.58 82.08) (width 1) (layer "B.Cu") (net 8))
 (segment (start 157 82.5) (end 157 96) (width 1) (layer "B.Cu") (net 8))
 (segment (start 135.5 102.5) (end 130.08 97.08) (width 1) (layer "B.Cu") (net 8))
 (segment (start 156.58 82.08) (end 157 82.5) (width 1) (layer "B.Cu") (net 8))
 (segment (start 159 97.5) (end 151.5 105) (width 1) (layer "B.Cu") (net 19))
 (segment (start 151.5 105) (end 127.5 105) (width 1) (layer "B.Cu") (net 19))
 (segment (start 158.54 79.54) (end 159 80) (width 1) (layer "B.Cu") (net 19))
 (segment (start 126.005 103.505) (end 124.66 103.505) (width 1) (layer "B.Cu") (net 19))
 (segment (start 127.5 105) (end 126.005 103.505) (width 1) (layer "B.Cu") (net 19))
 (segment (start 154 79.54) (end 158.54 79.54) (width 1) (layer "B.Cu") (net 19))
 (segment (start 159 80) (end 159 97.5) (width 1) (layer "B.Cu") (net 19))
 (segment (start 122 85) (end 122 86) (width 1) (layer "F.Cu") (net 9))
 (segment (start 122 86) (end 124.66 88.66) (width 1) (layer "F.Cu") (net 9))
 (segment (start 124.66 88.66) (end 124.66 99.06) (width 1) (layer "F.Cu") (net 9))
 (segment (start 125.22 99.62) (end 124.66 99.06) (width 1) (layer "B.Cu") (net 9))
 (segment (start 129 99.62) (end 125.22 99.62) (width 1) (layer "B.Cu") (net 9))
 (segment (start 124.66 99.06) (end 124.66 98.5075) (width 1) (layer "B.Cu") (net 9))
 (segment (start 124.66 98.5075) (end 122.1525 96) (width 1) (layer "B.Cu") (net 9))
 (segment (start 122.1525 96) (end 122 96) (width 1) (layer "B.Cu") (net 9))
 (segment (start 108.46 100) (end 108.46 102.11) (width 1) (layer "B.Cu") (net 18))
 (segment (start 108.46 102.11) (end 109.855 103.505) (width 1) (layer "B.Cu") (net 18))
 (segment (start 109.855 103.505) (end 114.5 103.505) (width 1) (layer "B.Cu") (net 18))
 (segment (start 143 75.285) (end 142.875 75.16) (width 1) (layer "F.Cu") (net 11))
 (segment (start 141 94.5) (end 141 83) (width 1) (layer "F.Cu") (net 11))
 (segment (start 141 83) (end 143 81) (width 1) (layer "F.Cu") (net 11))
 (segment (start 143 81) (end 143 75.285) (width 1) (layer "F.Cu") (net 11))
 (segment (start 143 75.285) (end 143 79.5) (width 1) (layer "B.Cu") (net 11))
 (segment (start 143 79.5) (end 110 79.5) (width 1) (layer "B.Cu") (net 11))
 (segment (start 135.89 75.16) (end 136 75.27) (width 1) (layer "B.Cu") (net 11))
 (segment (start 110 79.5) (end 110 75.49) (width 1) (layer "B.Cu") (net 11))
 (segment (start 142.875 75.16) (end 143 75.285) (width 1) (layer "B.Cu") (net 11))
 (segment (start 136.62 94.54) (end 140.96 94.54) (width 1) (layer "B.Cu") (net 11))
 (segment (start 140.96 94.54) (end 141 94.5) (width 1) (layer "B.Cu") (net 11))
 (segment (start 136 75.27) (end 136 79.5) (width 1) (layer "B.Cu") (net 11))
 (segment (start 110 75.49) (end 110.49 75) (width 1) (layer "B.Cu") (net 11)))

